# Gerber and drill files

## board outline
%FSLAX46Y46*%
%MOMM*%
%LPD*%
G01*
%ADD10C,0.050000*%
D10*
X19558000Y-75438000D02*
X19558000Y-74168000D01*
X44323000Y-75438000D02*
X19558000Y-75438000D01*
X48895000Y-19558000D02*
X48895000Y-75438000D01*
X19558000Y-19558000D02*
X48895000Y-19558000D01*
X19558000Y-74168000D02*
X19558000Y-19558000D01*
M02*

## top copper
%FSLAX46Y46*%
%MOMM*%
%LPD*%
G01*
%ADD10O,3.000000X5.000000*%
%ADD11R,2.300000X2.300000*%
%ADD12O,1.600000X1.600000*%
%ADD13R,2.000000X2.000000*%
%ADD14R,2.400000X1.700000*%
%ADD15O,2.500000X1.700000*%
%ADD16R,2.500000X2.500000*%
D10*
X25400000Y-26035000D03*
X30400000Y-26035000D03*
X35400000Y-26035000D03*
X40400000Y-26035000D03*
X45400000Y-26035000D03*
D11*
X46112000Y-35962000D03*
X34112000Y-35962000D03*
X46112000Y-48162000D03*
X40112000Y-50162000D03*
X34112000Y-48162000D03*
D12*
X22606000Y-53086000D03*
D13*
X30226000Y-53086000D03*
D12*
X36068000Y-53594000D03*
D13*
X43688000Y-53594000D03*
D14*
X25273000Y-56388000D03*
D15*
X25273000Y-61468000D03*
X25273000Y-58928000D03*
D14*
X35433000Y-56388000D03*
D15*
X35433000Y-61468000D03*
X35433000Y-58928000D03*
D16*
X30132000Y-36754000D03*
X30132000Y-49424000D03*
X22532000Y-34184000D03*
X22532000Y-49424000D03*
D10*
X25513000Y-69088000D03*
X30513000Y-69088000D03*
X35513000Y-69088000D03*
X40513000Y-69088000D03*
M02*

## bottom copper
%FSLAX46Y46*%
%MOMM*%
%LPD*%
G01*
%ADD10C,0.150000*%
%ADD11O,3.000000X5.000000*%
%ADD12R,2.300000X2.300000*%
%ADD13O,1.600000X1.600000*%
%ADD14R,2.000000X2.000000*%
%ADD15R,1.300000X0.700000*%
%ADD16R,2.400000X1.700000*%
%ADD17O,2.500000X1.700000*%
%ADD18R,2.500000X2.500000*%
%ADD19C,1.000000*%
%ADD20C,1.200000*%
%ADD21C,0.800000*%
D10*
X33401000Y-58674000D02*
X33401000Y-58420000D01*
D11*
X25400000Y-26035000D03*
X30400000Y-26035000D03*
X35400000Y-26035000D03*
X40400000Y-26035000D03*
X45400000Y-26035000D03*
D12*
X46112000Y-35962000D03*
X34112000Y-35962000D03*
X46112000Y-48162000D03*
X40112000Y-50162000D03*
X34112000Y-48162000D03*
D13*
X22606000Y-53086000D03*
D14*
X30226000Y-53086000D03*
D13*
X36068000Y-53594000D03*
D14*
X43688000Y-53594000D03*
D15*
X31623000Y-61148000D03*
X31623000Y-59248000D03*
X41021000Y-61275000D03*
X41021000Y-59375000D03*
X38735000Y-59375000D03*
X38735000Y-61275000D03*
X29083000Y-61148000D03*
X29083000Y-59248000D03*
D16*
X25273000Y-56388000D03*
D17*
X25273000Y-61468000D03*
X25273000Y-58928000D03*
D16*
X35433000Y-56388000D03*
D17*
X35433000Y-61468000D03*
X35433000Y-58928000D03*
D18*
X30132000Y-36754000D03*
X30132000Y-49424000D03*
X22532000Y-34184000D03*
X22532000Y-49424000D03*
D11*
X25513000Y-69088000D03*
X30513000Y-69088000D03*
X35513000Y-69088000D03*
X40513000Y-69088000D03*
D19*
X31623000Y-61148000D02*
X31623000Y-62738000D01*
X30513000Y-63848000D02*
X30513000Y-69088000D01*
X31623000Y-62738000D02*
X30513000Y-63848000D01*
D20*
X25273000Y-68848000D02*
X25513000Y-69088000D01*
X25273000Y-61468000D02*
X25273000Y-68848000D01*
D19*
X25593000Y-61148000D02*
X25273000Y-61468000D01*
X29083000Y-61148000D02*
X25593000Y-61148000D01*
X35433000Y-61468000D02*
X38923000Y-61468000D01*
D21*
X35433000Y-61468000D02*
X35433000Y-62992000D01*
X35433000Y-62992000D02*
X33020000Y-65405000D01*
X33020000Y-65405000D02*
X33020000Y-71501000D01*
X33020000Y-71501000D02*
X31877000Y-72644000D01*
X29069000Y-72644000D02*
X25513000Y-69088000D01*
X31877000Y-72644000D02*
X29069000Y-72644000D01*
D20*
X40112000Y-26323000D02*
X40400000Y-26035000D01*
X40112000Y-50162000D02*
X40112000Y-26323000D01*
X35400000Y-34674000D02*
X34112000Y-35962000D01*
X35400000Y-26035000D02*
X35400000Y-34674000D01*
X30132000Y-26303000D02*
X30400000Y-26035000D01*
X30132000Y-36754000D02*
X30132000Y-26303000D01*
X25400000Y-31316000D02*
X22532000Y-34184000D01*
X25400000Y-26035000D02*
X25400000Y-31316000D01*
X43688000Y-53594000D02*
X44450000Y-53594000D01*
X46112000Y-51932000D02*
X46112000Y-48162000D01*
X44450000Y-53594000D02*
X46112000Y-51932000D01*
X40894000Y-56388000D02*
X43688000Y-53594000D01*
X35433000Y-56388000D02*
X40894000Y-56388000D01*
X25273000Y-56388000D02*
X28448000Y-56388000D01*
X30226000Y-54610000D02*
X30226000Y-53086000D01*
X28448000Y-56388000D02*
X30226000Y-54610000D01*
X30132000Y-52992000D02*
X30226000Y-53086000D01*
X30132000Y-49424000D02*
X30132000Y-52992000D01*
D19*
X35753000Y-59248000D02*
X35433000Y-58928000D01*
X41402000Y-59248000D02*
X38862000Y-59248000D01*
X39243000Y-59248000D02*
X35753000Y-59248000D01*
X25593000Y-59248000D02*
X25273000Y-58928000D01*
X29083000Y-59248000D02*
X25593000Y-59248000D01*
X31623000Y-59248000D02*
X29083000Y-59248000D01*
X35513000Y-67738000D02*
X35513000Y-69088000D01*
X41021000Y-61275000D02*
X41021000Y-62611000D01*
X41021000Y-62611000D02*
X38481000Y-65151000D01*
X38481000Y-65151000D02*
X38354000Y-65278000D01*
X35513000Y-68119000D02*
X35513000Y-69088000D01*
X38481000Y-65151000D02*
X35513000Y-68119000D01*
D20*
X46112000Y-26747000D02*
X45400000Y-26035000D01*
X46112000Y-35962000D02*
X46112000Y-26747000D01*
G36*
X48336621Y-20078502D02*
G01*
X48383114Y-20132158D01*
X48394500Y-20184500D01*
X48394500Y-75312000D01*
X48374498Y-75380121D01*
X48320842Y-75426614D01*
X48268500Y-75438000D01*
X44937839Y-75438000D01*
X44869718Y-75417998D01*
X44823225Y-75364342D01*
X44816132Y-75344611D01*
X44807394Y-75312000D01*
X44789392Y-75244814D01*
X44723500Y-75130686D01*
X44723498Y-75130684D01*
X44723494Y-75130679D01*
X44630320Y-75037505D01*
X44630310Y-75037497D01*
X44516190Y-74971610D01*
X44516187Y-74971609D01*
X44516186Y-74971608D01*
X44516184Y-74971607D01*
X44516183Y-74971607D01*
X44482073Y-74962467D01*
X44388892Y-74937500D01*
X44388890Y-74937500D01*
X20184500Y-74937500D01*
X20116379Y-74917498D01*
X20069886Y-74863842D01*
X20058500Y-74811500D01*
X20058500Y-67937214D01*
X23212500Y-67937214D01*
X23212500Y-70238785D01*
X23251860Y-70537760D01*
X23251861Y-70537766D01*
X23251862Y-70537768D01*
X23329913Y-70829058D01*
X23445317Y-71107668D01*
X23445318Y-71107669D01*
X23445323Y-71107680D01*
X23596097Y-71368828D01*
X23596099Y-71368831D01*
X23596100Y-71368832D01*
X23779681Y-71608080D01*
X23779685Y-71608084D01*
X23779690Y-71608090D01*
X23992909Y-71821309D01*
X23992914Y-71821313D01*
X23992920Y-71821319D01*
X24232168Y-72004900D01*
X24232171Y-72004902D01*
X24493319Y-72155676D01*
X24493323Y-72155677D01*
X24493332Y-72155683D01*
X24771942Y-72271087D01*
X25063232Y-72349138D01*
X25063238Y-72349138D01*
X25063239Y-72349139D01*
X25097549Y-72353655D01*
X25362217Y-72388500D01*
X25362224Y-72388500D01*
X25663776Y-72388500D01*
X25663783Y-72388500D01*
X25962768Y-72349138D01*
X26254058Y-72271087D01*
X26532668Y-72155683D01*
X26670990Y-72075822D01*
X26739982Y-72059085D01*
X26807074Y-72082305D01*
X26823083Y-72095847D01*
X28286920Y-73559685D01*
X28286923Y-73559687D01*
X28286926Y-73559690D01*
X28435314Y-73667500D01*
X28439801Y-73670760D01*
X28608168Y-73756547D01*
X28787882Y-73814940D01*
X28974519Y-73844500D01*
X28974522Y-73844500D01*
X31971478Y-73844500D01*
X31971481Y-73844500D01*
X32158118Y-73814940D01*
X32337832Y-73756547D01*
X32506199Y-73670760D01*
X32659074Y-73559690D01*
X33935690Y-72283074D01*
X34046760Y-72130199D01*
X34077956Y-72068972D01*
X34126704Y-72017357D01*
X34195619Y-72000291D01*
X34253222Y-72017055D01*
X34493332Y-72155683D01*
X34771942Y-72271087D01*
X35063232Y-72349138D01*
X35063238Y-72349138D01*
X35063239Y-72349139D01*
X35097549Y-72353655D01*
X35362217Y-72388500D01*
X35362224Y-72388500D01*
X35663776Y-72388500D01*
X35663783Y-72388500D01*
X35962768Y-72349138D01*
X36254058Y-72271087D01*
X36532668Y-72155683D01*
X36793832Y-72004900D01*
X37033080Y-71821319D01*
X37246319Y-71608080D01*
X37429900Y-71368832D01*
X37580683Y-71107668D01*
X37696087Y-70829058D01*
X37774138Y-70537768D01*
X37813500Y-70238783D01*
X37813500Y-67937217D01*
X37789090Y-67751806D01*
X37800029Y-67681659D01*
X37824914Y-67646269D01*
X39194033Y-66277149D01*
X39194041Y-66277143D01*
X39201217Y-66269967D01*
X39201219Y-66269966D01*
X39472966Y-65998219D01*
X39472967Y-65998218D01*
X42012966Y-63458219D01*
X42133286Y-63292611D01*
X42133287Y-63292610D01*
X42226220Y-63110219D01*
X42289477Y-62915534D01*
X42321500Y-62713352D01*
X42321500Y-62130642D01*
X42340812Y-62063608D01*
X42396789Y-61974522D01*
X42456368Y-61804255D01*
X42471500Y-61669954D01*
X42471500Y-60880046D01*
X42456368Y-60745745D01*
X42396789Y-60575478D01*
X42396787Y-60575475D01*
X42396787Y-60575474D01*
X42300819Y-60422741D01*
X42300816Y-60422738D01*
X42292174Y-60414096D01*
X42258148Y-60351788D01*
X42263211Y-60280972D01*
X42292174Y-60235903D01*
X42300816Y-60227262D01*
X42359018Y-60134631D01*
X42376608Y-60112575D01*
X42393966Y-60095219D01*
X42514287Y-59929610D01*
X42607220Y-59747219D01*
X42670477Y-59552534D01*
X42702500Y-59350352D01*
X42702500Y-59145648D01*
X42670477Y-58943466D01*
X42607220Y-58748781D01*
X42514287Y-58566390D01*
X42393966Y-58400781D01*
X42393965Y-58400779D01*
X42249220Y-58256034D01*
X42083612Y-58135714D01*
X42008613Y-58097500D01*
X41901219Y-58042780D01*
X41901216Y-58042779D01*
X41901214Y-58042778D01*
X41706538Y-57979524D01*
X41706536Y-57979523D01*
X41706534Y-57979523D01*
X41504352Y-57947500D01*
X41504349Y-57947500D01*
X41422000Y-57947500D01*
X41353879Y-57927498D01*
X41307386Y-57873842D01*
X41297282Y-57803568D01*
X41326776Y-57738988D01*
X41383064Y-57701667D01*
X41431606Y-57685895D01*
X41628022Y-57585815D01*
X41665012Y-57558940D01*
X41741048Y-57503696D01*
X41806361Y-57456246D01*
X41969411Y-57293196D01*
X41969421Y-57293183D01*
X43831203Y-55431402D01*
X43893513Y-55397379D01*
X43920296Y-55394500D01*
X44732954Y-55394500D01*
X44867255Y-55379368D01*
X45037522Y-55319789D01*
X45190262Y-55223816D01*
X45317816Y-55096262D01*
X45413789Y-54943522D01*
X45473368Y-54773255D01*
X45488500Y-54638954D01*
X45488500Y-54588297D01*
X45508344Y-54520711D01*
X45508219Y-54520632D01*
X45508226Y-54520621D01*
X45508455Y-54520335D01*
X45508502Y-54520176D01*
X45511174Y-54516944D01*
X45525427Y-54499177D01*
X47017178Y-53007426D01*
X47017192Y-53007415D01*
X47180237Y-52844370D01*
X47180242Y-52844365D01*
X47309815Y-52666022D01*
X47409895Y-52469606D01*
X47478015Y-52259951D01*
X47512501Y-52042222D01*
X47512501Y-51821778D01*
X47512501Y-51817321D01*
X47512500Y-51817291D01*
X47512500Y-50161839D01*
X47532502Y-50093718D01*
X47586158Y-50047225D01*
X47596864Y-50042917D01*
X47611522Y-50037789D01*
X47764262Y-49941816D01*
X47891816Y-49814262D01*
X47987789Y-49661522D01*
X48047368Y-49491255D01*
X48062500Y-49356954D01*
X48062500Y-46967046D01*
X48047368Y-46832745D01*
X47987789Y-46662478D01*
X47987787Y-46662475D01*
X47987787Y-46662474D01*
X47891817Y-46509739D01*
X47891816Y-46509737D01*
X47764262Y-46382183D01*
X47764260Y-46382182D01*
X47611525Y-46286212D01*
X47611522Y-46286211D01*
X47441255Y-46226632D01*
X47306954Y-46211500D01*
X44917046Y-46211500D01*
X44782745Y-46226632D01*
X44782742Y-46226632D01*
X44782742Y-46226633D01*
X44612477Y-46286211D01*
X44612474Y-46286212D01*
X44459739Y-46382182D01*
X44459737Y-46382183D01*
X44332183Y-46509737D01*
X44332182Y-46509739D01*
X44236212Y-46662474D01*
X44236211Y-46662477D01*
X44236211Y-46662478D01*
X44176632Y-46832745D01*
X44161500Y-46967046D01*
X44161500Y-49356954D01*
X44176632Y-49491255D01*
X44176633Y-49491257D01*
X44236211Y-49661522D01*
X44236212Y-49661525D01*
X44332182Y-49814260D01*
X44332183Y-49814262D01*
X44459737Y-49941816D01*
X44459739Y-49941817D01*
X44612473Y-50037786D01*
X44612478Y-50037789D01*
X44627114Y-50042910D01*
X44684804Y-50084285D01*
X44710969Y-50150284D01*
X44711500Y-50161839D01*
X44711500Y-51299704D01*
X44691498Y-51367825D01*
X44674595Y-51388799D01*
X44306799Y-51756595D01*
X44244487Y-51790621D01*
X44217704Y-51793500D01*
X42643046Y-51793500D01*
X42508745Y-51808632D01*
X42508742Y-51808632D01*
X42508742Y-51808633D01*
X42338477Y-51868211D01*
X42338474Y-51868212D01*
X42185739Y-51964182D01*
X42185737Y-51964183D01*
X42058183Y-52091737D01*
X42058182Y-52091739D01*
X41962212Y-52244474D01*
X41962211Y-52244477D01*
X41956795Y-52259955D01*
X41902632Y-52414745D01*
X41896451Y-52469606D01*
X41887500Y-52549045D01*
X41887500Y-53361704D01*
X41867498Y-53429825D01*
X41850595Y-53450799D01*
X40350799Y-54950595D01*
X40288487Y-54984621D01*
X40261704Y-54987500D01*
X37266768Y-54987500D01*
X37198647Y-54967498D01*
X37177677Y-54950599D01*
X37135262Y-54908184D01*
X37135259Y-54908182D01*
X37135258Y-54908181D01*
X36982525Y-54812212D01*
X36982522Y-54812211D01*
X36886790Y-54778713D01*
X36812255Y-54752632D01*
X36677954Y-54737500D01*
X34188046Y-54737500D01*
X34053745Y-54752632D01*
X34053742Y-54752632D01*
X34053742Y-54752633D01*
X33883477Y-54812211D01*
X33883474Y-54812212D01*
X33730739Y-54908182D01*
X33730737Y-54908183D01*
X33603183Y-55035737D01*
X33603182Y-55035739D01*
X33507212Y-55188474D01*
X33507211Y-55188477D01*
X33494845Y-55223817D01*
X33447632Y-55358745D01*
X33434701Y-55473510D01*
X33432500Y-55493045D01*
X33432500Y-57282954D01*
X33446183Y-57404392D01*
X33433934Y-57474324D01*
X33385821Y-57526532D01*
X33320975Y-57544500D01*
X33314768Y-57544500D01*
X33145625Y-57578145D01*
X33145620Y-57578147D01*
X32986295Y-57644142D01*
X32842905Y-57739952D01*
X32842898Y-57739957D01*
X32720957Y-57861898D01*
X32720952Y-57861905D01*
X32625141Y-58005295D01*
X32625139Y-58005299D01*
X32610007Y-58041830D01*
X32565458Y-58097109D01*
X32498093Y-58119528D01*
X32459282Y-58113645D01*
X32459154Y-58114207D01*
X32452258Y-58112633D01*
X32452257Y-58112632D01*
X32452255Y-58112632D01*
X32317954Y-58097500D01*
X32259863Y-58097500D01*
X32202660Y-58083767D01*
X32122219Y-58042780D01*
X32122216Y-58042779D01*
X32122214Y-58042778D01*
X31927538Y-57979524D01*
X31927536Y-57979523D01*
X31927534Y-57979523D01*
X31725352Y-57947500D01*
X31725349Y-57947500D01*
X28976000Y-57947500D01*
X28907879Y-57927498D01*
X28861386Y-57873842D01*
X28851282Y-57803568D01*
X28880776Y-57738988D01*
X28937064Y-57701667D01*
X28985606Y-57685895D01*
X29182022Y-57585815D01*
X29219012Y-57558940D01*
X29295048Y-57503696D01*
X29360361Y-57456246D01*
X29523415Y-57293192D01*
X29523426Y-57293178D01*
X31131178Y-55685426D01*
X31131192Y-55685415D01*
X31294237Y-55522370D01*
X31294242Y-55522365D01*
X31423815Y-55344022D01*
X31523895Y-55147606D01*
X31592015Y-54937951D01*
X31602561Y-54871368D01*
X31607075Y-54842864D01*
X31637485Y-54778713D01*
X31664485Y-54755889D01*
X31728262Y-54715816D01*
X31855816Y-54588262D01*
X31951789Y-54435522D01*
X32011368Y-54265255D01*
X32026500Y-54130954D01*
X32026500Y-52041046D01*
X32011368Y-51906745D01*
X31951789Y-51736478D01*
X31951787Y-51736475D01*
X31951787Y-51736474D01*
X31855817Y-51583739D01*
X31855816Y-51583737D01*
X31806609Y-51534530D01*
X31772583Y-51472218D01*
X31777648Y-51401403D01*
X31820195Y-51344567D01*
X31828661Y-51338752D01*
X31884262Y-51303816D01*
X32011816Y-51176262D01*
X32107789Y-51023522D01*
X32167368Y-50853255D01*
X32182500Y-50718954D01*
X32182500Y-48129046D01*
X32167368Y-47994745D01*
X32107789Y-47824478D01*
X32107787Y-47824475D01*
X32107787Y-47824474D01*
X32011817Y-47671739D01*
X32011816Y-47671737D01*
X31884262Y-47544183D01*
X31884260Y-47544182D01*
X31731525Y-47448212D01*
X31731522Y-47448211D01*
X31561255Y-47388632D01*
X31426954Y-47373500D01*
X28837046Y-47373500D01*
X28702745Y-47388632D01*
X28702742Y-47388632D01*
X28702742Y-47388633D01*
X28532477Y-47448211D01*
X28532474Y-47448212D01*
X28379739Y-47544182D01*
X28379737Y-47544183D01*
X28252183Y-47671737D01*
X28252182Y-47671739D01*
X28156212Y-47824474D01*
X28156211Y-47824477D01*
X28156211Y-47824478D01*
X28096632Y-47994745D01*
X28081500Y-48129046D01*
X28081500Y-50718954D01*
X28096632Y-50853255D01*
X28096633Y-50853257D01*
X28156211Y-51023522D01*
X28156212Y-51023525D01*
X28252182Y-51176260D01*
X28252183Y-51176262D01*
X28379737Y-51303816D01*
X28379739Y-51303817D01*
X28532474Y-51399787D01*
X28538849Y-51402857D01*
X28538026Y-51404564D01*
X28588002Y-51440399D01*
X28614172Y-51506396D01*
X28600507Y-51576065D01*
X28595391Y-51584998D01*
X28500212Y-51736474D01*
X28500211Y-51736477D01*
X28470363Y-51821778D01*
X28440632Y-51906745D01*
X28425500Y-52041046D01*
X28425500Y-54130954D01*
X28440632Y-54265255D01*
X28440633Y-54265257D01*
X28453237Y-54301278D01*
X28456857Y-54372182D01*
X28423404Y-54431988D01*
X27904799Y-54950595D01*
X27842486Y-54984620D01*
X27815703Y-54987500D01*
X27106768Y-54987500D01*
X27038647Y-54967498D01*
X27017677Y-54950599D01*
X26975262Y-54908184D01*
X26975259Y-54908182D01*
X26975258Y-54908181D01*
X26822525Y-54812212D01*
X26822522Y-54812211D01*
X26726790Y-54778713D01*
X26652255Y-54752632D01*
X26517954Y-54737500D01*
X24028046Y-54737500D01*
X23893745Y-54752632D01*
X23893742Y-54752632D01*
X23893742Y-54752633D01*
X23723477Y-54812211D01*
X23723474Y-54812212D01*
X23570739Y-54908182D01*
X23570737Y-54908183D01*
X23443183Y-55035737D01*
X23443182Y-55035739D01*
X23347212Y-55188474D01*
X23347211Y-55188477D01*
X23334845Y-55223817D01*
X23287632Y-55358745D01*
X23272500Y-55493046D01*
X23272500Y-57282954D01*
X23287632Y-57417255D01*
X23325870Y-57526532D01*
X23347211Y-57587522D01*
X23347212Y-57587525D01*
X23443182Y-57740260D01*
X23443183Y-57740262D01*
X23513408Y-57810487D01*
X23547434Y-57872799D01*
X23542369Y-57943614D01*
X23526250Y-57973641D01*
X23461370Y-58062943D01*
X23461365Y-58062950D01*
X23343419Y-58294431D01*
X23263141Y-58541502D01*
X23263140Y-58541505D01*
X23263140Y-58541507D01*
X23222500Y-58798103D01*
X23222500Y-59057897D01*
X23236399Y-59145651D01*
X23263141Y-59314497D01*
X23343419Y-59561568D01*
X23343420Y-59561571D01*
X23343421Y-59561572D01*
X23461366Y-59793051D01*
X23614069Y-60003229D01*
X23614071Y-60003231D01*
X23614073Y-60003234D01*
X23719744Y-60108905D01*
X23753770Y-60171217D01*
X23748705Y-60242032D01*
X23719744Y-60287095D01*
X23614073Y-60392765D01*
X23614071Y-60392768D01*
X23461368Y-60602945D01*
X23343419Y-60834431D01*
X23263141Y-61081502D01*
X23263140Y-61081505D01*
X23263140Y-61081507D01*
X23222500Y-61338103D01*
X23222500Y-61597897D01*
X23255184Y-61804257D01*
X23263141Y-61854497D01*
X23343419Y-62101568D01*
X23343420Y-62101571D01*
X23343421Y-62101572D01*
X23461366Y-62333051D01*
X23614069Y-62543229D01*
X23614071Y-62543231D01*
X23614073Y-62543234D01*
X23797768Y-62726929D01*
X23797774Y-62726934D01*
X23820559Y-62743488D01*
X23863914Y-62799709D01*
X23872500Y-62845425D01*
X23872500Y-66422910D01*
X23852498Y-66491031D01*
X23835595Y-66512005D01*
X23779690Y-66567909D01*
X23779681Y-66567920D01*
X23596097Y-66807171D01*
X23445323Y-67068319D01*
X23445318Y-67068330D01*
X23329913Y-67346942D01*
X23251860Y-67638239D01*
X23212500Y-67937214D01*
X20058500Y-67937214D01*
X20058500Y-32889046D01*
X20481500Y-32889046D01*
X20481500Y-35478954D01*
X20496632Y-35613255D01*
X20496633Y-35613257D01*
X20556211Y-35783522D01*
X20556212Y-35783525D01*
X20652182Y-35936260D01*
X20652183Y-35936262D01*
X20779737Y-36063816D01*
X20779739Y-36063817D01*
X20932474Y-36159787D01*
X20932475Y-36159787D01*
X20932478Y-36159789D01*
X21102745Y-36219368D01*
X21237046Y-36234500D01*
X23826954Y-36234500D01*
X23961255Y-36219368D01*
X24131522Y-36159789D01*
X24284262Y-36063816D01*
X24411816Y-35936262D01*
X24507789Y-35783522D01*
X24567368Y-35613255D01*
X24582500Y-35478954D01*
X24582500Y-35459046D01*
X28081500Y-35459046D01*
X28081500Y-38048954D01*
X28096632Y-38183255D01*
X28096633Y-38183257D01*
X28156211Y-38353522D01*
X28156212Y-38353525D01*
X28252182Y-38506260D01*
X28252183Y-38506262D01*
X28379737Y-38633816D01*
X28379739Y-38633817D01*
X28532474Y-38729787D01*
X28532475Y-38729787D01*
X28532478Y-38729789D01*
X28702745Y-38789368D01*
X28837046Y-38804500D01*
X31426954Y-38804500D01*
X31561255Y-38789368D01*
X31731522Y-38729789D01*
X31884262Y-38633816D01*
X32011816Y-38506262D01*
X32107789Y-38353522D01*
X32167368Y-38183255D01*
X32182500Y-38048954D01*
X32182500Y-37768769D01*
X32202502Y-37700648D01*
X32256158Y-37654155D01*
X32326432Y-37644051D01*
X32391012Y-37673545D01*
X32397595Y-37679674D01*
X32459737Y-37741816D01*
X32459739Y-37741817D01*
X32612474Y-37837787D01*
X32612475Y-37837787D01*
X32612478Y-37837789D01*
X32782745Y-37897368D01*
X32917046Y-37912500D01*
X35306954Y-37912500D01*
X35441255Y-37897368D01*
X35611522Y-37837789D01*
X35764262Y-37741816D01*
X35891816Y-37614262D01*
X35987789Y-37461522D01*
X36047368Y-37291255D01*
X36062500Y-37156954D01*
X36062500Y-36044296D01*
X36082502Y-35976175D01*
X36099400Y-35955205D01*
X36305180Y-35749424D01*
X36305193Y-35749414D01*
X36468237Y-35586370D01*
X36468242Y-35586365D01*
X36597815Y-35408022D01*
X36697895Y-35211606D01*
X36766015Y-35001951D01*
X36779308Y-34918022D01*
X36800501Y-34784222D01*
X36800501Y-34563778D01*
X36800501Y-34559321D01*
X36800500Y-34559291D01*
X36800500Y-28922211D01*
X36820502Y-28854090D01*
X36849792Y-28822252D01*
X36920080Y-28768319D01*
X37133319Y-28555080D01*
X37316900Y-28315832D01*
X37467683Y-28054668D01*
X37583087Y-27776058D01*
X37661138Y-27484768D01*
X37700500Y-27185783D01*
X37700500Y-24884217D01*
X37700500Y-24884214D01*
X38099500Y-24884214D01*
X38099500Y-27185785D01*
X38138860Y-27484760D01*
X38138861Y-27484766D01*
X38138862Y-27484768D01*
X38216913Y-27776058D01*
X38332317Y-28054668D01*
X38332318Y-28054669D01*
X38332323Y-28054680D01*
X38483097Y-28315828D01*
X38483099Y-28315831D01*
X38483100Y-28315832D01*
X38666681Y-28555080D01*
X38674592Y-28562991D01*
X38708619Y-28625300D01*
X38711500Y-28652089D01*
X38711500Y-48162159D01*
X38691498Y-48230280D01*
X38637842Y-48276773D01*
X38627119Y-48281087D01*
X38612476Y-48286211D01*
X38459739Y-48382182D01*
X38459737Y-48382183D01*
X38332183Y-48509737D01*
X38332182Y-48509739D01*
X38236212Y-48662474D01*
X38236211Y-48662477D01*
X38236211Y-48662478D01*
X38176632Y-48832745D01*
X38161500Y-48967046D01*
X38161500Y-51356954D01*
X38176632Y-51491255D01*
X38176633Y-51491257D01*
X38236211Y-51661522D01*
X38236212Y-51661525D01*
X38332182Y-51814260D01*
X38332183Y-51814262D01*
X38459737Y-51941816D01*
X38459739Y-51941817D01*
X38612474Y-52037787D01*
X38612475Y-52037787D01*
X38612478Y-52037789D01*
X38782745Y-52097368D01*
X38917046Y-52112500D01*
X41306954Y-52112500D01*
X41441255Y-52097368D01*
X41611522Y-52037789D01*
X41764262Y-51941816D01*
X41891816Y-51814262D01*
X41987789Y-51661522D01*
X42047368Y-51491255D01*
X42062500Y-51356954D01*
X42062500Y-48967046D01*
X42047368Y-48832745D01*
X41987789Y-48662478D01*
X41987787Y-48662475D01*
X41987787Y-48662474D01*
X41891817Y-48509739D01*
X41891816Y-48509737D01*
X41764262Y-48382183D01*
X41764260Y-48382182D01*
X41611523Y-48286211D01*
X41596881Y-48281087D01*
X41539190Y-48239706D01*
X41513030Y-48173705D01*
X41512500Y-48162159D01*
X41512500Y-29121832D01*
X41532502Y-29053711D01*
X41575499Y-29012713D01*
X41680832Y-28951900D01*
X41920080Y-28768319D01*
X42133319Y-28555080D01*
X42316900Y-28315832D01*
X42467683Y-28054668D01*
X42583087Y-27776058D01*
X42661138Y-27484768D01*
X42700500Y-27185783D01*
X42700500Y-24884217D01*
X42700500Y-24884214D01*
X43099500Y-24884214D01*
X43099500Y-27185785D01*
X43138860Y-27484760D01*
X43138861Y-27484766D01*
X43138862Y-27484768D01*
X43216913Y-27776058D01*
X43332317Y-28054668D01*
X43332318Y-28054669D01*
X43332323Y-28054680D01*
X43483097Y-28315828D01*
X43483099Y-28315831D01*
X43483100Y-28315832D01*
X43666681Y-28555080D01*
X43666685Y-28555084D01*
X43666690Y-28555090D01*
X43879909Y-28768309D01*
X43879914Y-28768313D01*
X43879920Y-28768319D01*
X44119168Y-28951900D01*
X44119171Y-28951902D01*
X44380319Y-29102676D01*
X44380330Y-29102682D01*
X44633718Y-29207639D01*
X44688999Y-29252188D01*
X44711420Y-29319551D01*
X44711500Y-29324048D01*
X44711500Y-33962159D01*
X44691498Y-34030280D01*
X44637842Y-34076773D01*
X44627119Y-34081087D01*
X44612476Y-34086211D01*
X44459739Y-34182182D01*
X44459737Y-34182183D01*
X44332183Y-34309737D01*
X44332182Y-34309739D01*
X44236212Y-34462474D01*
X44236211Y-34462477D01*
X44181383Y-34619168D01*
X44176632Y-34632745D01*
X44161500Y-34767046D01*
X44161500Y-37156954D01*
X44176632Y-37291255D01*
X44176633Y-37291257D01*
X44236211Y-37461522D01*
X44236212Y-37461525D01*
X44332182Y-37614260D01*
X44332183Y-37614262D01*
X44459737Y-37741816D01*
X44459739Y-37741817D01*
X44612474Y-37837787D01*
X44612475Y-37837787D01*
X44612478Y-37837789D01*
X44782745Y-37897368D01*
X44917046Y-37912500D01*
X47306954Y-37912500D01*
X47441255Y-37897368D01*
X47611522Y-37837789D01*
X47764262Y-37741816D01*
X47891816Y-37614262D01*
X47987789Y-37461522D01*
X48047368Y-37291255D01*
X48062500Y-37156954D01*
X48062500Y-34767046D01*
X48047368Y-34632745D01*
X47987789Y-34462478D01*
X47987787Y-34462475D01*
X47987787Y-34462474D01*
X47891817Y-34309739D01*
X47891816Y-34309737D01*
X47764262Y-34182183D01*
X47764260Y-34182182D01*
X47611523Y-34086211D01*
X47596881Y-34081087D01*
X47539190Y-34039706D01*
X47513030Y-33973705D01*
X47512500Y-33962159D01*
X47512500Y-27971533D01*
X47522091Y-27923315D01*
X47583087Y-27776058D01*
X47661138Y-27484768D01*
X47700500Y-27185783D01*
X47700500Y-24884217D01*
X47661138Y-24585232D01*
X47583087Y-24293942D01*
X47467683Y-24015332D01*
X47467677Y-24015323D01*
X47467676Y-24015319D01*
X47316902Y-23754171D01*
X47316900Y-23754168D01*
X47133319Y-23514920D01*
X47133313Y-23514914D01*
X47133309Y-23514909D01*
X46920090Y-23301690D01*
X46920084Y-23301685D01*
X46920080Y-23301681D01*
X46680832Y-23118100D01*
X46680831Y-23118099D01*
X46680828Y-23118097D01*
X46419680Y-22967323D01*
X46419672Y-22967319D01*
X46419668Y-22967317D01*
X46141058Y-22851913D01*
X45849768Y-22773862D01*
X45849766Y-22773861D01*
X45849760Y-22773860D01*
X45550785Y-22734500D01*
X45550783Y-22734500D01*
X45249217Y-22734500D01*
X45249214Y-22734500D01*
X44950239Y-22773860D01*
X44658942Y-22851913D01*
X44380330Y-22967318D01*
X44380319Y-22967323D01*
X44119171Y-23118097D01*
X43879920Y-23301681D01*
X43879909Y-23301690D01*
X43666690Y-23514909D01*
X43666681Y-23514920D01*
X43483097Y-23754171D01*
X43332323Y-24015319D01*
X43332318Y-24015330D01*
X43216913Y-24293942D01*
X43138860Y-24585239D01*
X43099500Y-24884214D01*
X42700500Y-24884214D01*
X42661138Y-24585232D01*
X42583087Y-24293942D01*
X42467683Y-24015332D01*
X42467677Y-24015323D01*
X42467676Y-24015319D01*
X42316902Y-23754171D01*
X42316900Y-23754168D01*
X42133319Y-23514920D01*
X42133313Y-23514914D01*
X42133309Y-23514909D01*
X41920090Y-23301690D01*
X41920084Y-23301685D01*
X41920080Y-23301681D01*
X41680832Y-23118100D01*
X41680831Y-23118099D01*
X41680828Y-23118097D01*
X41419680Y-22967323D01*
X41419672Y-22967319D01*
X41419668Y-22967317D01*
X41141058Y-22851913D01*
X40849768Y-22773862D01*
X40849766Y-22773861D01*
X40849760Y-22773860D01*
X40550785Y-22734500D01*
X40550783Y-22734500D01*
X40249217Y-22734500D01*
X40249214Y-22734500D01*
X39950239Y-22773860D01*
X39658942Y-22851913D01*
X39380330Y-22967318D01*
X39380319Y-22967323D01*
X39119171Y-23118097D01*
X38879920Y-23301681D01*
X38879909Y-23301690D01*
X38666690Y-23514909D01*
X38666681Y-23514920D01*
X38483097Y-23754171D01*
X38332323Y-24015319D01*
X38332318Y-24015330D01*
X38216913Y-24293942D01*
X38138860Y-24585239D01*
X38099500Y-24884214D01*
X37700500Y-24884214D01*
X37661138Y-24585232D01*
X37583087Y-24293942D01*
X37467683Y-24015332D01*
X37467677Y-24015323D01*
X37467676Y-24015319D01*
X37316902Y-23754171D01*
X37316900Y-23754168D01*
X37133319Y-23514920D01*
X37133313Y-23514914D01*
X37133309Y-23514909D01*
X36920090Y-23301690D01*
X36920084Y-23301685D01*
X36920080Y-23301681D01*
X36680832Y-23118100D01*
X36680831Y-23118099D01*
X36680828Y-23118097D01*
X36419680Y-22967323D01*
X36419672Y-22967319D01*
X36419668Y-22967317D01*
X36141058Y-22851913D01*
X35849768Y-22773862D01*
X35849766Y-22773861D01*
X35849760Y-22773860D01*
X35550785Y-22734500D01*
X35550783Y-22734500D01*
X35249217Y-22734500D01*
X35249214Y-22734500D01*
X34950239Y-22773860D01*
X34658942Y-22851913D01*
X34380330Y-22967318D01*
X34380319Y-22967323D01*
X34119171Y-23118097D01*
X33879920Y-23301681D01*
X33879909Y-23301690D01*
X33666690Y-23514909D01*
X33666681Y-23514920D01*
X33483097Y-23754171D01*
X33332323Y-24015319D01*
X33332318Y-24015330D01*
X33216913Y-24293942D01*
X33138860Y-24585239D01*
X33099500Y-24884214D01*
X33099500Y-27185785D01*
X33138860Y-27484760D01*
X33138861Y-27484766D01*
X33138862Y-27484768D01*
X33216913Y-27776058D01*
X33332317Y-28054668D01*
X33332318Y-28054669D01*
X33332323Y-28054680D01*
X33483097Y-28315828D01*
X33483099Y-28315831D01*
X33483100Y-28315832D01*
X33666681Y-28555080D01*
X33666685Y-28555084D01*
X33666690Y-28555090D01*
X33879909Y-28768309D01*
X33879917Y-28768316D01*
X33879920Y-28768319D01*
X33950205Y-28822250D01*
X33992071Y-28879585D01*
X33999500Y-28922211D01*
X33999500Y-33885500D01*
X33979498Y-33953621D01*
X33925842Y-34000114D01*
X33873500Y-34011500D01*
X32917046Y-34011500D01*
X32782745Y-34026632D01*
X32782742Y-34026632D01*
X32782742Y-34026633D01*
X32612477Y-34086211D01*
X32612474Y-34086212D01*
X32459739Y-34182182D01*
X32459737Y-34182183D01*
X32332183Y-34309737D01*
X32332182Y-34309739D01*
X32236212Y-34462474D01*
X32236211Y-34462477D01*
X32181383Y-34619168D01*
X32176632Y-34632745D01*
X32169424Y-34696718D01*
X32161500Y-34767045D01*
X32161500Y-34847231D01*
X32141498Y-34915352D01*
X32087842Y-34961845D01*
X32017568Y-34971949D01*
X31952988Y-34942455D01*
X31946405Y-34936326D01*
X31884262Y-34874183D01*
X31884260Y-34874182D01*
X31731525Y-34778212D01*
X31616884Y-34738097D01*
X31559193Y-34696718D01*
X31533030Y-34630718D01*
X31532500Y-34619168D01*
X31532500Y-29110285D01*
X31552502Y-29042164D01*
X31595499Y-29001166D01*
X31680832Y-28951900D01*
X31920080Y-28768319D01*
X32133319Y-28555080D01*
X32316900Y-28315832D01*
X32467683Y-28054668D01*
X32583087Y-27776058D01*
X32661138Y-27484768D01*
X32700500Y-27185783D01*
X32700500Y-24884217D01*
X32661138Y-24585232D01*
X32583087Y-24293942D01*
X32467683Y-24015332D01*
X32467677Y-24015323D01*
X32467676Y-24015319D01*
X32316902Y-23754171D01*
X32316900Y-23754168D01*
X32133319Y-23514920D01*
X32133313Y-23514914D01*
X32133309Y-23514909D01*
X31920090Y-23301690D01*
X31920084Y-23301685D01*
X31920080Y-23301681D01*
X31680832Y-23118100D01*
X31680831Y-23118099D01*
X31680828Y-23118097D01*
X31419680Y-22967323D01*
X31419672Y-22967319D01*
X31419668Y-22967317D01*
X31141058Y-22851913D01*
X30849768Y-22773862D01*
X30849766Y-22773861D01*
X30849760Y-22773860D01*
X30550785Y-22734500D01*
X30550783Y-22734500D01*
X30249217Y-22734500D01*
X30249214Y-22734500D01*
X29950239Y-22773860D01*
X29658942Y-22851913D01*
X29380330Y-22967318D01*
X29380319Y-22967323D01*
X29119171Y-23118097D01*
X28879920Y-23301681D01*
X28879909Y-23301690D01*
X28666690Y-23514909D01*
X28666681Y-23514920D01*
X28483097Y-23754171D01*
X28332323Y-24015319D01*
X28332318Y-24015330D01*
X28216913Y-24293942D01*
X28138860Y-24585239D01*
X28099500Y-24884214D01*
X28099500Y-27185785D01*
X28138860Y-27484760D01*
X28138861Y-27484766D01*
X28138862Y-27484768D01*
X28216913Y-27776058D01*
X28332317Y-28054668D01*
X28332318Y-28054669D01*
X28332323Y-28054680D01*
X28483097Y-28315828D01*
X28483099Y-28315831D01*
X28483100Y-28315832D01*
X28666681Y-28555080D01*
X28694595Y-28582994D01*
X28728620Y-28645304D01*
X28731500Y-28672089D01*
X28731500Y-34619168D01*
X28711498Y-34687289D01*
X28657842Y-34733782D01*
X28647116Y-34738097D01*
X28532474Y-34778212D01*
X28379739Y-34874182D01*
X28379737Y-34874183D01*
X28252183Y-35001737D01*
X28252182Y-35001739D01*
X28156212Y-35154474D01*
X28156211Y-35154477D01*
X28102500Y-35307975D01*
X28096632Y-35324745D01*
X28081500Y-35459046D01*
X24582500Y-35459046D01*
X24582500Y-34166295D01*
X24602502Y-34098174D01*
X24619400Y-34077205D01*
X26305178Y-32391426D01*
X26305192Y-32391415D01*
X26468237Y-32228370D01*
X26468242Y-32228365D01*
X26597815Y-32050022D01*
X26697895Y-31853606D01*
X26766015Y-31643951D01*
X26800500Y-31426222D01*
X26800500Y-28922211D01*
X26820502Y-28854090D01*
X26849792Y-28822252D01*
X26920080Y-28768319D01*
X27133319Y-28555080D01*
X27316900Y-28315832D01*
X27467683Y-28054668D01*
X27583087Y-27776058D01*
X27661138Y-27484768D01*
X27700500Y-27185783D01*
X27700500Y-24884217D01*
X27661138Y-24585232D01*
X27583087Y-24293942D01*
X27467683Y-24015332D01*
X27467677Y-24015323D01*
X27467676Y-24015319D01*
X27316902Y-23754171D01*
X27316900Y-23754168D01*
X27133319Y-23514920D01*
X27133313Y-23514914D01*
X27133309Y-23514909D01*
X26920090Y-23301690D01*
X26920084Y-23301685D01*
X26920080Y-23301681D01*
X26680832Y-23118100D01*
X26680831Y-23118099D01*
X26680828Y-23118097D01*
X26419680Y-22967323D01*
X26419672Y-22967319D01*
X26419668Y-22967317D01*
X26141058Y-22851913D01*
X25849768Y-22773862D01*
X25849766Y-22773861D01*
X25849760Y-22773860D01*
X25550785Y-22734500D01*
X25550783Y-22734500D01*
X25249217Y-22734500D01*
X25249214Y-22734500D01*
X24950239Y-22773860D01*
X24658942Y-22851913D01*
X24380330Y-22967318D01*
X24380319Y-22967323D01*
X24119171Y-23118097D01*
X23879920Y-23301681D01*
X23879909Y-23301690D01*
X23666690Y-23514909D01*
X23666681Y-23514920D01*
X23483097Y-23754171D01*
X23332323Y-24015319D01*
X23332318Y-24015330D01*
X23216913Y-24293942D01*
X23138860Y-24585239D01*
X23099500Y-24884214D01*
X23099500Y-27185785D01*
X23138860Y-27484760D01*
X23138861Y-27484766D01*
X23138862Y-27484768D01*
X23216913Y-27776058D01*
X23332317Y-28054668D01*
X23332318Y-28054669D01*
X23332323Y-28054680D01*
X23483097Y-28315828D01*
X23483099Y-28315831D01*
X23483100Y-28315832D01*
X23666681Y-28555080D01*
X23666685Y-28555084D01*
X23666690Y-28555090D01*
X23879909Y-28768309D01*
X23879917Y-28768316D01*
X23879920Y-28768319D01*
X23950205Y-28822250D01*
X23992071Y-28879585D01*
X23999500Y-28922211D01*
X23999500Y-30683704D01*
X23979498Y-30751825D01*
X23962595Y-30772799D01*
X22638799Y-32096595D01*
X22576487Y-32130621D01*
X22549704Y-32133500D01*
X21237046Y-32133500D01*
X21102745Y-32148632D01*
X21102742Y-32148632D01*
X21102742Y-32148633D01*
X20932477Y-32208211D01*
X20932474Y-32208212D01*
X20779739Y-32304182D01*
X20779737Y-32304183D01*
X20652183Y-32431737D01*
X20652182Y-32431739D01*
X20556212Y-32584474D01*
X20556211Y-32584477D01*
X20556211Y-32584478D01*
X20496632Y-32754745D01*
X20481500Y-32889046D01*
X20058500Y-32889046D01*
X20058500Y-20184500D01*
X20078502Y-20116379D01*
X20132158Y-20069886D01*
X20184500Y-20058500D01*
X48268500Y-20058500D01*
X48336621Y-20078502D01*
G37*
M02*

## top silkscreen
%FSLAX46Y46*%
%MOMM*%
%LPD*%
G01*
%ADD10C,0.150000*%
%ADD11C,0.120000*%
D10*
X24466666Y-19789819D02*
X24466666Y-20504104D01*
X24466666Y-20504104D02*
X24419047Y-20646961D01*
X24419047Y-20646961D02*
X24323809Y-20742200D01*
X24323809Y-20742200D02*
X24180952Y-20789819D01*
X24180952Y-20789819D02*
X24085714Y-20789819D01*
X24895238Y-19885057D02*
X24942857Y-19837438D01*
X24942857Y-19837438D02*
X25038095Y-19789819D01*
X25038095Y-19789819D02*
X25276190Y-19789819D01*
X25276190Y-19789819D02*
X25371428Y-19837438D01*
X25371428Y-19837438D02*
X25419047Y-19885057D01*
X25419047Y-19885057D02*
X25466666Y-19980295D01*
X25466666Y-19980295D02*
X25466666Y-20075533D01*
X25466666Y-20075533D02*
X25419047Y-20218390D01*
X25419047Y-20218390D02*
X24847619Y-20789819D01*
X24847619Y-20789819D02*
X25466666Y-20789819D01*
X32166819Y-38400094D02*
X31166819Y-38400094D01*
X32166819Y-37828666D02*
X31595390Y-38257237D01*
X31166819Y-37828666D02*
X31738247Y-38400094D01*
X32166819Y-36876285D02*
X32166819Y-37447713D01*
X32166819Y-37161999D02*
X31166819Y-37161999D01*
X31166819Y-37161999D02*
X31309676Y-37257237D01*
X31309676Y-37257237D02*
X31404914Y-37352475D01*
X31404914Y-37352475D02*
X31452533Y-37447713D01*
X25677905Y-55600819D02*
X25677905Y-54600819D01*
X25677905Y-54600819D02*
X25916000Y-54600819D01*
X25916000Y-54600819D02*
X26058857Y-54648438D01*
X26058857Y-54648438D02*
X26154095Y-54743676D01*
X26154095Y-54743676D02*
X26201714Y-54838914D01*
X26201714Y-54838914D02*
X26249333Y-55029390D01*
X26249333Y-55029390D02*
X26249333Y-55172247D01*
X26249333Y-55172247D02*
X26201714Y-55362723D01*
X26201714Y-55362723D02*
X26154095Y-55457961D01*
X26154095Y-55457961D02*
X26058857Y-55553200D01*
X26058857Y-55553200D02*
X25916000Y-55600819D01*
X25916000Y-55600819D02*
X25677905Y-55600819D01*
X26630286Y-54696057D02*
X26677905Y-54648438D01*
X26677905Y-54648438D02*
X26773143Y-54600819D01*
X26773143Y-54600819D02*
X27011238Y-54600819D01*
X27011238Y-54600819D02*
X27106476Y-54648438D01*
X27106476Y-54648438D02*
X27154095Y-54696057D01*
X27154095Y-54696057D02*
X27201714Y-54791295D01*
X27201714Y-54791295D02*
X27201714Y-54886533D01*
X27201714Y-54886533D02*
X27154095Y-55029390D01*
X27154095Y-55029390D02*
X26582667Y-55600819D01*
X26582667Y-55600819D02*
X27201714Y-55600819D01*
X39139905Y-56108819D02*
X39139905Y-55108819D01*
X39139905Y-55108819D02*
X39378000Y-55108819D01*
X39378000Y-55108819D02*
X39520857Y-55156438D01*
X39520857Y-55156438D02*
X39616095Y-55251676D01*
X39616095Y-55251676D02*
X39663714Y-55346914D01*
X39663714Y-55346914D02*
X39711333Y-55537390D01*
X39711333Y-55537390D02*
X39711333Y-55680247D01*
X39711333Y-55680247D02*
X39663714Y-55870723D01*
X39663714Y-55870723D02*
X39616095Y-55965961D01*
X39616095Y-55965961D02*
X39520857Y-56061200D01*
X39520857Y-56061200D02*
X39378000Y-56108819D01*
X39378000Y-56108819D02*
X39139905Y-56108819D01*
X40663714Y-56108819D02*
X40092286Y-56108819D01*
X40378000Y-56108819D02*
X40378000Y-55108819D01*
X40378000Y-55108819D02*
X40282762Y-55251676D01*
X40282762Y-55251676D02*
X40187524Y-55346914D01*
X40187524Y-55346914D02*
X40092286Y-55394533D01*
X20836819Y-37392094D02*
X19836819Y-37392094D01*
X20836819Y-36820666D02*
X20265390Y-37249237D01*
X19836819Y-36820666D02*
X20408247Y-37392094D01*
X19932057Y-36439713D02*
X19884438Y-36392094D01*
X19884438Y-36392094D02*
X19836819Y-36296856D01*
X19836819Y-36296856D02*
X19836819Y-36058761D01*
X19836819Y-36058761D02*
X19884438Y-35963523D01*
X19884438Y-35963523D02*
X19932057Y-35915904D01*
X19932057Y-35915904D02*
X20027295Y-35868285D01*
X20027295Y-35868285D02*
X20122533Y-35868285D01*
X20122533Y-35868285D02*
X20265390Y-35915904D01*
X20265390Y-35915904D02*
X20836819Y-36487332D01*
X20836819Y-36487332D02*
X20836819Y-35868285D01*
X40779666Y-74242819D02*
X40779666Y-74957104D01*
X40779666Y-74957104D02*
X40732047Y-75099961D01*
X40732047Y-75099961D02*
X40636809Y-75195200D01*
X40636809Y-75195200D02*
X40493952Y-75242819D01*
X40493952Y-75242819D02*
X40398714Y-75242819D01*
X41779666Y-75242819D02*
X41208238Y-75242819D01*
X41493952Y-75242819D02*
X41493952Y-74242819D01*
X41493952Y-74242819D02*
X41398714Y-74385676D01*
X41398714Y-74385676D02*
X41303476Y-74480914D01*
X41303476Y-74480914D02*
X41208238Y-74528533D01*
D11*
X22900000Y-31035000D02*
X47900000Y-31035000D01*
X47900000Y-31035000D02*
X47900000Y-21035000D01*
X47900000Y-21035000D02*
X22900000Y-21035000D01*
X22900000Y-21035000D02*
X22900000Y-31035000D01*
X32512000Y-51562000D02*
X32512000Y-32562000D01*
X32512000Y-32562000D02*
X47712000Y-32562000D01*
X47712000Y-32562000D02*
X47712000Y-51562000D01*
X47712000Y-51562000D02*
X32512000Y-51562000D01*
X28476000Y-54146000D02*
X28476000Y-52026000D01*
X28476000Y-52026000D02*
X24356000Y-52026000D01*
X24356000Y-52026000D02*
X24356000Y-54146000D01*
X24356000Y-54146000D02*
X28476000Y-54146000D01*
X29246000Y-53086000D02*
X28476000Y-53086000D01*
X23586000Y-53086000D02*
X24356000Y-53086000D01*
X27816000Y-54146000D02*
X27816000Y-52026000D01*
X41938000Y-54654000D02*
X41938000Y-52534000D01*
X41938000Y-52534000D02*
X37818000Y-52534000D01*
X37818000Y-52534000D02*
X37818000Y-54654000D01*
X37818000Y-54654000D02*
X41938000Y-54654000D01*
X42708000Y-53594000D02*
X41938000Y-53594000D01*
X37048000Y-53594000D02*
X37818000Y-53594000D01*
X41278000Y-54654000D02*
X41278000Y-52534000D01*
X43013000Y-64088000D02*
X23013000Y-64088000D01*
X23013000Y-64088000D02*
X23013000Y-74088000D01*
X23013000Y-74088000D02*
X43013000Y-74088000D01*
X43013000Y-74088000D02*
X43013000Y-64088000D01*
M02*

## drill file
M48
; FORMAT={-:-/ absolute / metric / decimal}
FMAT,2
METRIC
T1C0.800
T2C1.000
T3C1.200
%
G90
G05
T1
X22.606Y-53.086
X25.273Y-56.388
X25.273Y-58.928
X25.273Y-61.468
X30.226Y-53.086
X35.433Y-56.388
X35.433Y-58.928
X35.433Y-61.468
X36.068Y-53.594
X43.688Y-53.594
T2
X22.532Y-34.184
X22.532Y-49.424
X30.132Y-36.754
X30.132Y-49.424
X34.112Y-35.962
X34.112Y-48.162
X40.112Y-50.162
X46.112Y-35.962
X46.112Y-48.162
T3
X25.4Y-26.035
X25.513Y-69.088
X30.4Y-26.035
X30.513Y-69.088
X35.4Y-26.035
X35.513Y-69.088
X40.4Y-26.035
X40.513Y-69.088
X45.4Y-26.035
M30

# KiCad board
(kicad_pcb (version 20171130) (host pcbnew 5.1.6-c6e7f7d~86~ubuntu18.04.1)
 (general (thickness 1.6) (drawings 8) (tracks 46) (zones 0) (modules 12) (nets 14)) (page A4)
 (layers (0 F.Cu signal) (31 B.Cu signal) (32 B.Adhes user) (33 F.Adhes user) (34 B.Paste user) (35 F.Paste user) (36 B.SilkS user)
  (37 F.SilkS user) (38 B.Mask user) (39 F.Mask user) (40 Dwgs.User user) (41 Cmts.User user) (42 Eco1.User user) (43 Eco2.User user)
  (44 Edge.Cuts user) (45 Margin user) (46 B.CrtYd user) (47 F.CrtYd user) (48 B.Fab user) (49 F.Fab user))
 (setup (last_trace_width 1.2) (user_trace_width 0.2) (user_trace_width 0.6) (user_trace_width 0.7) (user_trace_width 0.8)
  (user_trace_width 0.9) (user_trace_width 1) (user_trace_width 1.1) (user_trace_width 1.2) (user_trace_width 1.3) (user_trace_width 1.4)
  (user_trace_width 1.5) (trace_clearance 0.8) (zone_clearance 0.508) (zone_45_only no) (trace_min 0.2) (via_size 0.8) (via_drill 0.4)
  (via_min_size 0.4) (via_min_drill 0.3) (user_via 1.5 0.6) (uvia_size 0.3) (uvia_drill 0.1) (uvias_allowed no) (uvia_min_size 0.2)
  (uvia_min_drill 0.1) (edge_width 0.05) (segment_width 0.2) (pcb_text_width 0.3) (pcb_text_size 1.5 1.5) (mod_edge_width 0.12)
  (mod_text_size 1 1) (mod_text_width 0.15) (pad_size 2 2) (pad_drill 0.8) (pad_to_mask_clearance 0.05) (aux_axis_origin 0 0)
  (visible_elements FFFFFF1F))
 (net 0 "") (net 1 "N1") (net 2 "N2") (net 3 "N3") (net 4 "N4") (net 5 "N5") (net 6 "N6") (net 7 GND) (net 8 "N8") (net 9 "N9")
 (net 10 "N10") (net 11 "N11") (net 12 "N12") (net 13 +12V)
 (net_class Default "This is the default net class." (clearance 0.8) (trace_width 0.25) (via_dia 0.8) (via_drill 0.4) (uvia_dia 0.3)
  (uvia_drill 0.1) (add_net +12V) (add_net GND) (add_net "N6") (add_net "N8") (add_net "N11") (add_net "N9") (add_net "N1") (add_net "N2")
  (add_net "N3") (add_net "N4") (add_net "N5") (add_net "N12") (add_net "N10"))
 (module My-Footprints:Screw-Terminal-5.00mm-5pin (layer F.Cu) (at 25.4 26.035)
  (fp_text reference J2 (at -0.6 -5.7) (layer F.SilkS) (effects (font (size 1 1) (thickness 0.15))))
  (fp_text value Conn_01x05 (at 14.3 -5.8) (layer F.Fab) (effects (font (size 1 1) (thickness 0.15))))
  (fp_line (start -2.5 5) (end 22.5 5) (layer F.SilkS) (width 0.12))
  (fp_line (start 22.5 5) (end 22.5 -5) (layer F.SilkS) (width 0.12))
  (fp_line (start 22.5 -5) (end -2.5 -5) (layer F.SilkS) (width 0.12))
  (fp_line (start -2.5 -5) (end -2.5 5) (layer F.SilkS) (width 0.12))
  (pad 1 thru_hole oval (at 0 0 90) (size 5 3) (drill 1.2) (layers *.Cu *.Mask) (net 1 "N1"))
  (pad 2 thru_hole oval (at 5 0 90) (size 5 3) (drill 1.2) (layers *.Cu *.Mask) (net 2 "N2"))
  (pad 3 thru_hole oval (at 10 0 90) (size 5 3) (drill 1.2) (layers *.Cu *.Mask) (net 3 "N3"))
  (pad 4 thru_hole oval (at 15 0 90) (size 5 3) (drill 1.2) (layers *.Cu *.Mask) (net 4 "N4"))
  (pad 5 thru_hole oval (at 20 0 90) (size 5 3) (drill 1.2) (layers *.Cu *.Mask) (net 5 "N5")))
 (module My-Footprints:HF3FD (layer F.Cu) (at 32.512 51.562 90)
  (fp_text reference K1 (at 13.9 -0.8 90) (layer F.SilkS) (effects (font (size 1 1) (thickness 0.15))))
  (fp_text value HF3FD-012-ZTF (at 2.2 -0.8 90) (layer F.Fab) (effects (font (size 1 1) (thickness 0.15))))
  (fp_line (start 0 0) (end 19 0) (layer F.SilkS) (width 0.12))
  (fp_line (start 19 0) (end 19 15.2) (layer F.SilkS) (width 0.12))
  (fp_line (start 19 15.2) (end 0 15.2) (layer F.SilkS) (width 0.12))
  (fp_line (start 0 15.2) (end 0 0) (layer F.SilkS) (width 0.12))
  (pad NC thru_hole rect (at 15.6 13.6 90) (size 2.3 2.3) (drill 1) (layers *.Cu *.Mask) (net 5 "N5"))
  (pad NO thru_hole rect (at 15.6 1.6 90) (size 2.3 2.3) (drill 1) (layers *.Cu *.Mask) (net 3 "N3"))
  (pad C2 thru_hole rect (at 3.4 13.6 90) (size 2.3 2.3) (drill 1) (layers *.Cu *.Mask) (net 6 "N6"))
  (pad COM thru_hole rect (at 1.4 7.6 90) (size 2.3 2.3) (drill 1) (layers *.Cu *.Mask) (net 4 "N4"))
  (pad C1 thru_hole rect (at 3.4 1.6 90) (size 2.3 2.3) (drill 1) (layers *.Cu *.Mask) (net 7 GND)))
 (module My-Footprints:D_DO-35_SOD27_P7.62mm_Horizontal (layer F.Cu) (at 30.226 53.086 180)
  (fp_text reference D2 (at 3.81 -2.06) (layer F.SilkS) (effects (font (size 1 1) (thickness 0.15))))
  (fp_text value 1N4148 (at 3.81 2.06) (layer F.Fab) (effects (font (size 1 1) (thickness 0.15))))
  (fp_line (start 1.75 -1.06) (end 1.75 1.06) (layer F.SilkS) (width 0.12))
  (fp_line (start 1.75 1.06) (end 5.87 1.06) (layer F.SilkS) (width 0.12))
  (fp_line (start 5.87 1.06) (end 5.87 -1.06) (layer F.SilkS) (width 0.12))
  (fp_line (start 5.87 -1.06) (end 1.75 -1.06) (layer F.SilkS) (width 0.12))
  (fp_line (start 0.98 0) (end 1.75 0) (layer F.SilkS) (width 0.12))
  (fp_line (start 6.64 0) (end 5.87 0) (layer F.SilkS) (width 0.12))
  (fp_line (start 2.41 -1.06) (end 2.41 1.06) (layer F.SilkS) (width 0.12))
  (pad A thru_hole oval (at 7.62 0 180) (size 1.6 1.6) (drill 0.8) (layers *.Cu *.Mask) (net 7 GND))
  (pad C thru_hole rect (at 0 0 180) (size 2 2) (drill 0.8) (layers *.Cu *.Mask) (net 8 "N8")))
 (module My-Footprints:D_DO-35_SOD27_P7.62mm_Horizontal (layer F.Cu) (at 43.688 53.594 180)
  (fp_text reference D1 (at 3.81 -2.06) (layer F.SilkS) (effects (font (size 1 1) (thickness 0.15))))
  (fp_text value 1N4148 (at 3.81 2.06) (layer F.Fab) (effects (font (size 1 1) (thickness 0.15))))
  (fp_line (start 1.75 -1.06) (end 1.75 1.06) (layer F.SilkS) (width 0.12))
  (fp_line (start 1.75 1.06) (end 5.87 1.06) (layer F.SilkS) (width 0.12))
  (fp_line (start 5.87 1.06) (end 5.87 -1.06) (layer F.SilkS) (width 0.12))
  (fp_line (start 5.87 -1.06) (end 1.75 -1.06) (layer F.SilkS) (width 0.12))
  (fp_line (start 0.98 0) (end 1.75 0) (layer F.SilkS) (width 0.12))
  (fp_line (start 6.64 0) (end 5.87 0) (layer F.SilkS) (width 0.12))
  (fp_line (start 2.41 -1.06) (end 2.41 1.06) (layer F.SilkS) (width 0.12))
  (pad A thru_hole oval (at 7.62 0 180) (size 1.6 1.6) (drill 0.8) (layers *.Cu *.Mask) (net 7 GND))
  (pad C thru_hole rect (at 0 0 180) (size 2 2) (drill 0.8) (layers *.Cu *.Mask) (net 6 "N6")))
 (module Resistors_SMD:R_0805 (layer B.Cu) (at 31.623 60.198 90)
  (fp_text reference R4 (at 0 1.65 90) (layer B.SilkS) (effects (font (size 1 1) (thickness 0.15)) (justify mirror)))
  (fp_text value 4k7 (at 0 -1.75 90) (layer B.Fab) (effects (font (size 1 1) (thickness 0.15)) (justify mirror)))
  (pad 1 smd rect (at -0.95 0 90) (size 0.7 1.3) (layers B.Cu B.Paste B.Mask) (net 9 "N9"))
  (pad 2 smd rect (at 0.95 0 90) (size 0.7 1.3) (layers B.Cu B.Paste B.Mask) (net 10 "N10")))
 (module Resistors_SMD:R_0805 (layer B.Cu) (at 41.021 60.325 90)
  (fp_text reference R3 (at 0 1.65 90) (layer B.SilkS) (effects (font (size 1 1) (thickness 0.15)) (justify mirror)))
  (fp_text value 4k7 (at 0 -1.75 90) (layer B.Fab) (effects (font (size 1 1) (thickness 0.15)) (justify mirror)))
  (pad 1 smd rect (at -0.95 0 90) (size 0.7 1.3) (layers B.Cu B.Paste B.Mask) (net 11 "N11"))
  (pad 2 smd rect (at 0.95 0 90) (size 0.7 1.3) (layers B.Cu B.Paste B.Mask) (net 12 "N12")))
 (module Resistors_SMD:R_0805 (layer B.Cu) (at 38.735 60.325 270)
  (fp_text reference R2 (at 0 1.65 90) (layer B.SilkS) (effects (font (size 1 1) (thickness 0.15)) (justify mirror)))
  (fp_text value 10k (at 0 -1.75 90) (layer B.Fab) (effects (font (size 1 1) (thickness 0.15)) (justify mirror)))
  (pad 1 smd rect (at -0.95 0 270) (size 0.7 1.3) (layers B.Cu B.Paste B.Mask) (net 12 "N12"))
  (pad 2 smd rect (at 0.95 0 270) (size 0.7 1.3) (layers B.Cu B.Paste B.Mask) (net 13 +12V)))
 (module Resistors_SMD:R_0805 (layer B.Cu) (at 29.083 60.198 90)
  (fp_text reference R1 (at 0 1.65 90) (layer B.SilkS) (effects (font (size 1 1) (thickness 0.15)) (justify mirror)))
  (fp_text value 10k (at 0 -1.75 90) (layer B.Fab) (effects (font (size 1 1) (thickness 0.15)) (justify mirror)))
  (pad 1 smd rect (at -0.95 0 90) (size 0.7 1.3) (layers B.Cu B.Paste B.Mask) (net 13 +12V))
  (pad 2 smd rect (at 0.95 0 90) (size 0.7 1.3) (layers B.Cu B.Paste B.Mask) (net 10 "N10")))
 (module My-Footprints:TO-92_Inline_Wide (layer B.Cu) (at 25.273 56.388 270)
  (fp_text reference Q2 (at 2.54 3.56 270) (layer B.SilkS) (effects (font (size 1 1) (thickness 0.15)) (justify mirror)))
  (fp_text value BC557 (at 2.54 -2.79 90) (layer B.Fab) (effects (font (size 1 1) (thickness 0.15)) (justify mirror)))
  (pad 1 thru_hole rect (at 0 0 180) (size 2.4 1.7) (drill 0.8) (layers *.Cu *.Mask) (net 8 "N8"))
  (pad 3 thru_hole oval (at 5.08 0 180) (size 2.5 1.7) (drill 0.8) (layers *.Cu *.Mask) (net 13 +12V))
  (pad 2 thru_hole oval (at 2.54 0 180) (size 2.5 1.7) (drill 0.8) (layers *.Cu *.Mask) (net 10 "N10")))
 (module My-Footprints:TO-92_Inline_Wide (layer B.Cu) (at 35.433 56.388 270)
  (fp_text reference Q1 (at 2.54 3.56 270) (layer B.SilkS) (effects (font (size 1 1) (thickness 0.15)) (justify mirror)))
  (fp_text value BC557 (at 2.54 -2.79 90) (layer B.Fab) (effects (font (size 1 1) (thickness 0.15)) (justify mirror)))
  (pad 1 thru_hole rect (at 0 0 180) (size 2.4 1.7) (drill 0.8) (layers *.Cu *.Mask) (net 6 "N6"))
  (pad 3 thru_hole oval (at 5.08 0 180) (size 2.5 1.7) (drill 0.8) (layers *.Cu *.Mask) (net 13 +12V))
  (pad 2 thru_hole oval (at 2.54 0 180) (size 2.5 1.7) (drill 0.8) (layers *.Cu *.Mask) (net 12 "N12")))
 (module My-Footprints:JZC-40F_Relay (layer F.Cu) (at 21.082 51.054 90)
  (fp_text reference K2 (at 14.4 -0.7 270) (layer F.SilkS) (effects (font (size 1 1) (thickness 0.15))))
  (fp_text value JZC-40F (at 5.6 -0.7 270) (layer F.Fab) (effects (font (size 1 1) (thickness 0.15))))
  (pad 4 thru_hole rect (at 14.3 9.05 90) (size 2.5 2.5) (drill 1) (layers *.Cu *.Mask) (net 2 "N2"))
  (pad 1 thru_hole rect (at 1.63 9.05 90) (size 2.5 2.5) (drill 1) (layers *.Cu *.Mask) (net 8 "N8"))
  (pad 3 thru_hole rect (at 16.87 1.45 90) (size 2.5 2.5) (drill 1) (layers *.Cu *.Mask) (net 1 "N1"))
  (pad 2 thru_hole rect (at 1.63 1.45 90) (size 2.5 2.5) (drill 1) (layers *.Cu *.Mask) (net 7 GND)))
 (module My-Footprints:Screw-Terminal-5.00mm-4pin (layer F.Cu) (at 40.513 69.088 180)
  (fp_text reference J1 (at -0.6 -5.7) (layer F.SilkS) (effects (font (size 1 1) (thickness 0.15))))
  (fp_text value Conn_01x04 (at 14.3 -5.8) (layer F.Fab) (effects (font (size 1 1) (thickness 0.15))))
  (fp_line (start -2.5 5) (end 17.5 5) (layer F.SilkS) (width 0.12))
  (fp_line (start 17.5 5) (end 17.5 -5) (layer F.SilkS) (width 0.12))
  (fp_line (start 17.5 -5) (end -2.5 -5) (layer F.SilkS) (width 0.12))
  (fp_line (start -2.5 -5) (end -2.5 5) (layer F.SilkS) (width 0.12))
  (pad 4 thru_hole oval (at 15 0 270) (size 5 3) (drill 1.2) (layers *.Cu *.Mask) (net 13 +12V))
  (pad 3 thru_hole oval (at 10 0 270) (size 5 3) (drill 1.2) (layers *.Cu *.Mask) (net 9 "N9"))
  (pad 2 thru_hole oval (at 5 0 270) (size 5 3) (drill 1.2) (layers *.Cu *.Mask) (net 11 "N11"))
  (pad 1 thru_hole oval (at 0 0 270) (size 5 3) (drill 1.2) (layers *.Cu *.Mask) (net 7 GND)))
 (gr_line (start 33.401 58.674) (end 33.401 58.42) (layer B.Cu) (width 0.15))
 (gr_line (start 19.558 75.438) (end 19.558 74.168) (layer Edge.Cuts) (width 0.05))
 (gr_line (start 44.323 75.438) (end 19.558 75.438) (layer Edge.Cuts) (width 0.05))
 (gr_line (start 48.895 19.558) (end 48.895 75.438) (layer Edge.Cuts) (width 0.05))
 (gr_line (start 19.558 19.558) (end 48.895 19.558) (layer Edge.Cuts) (width 0.05))
 (gr_line (start 19.558 74.168) (end 19.558 19.558) (layer Edge.Cuts) (width 0.05))
 (segment (start 31.623 61.148) (end 31.623 62.738) (width 1) (layer B.Cu) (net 9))
 (segment (start 30.513 63.848) (end 30.513 69.088) (width 1) (layer B.Cu) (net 9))
 (segment (start 31.623 62.738) (end 30.513 63.848) (width 1) (layer B.Cu) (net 9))
 (segment (start 25.273 68.848) (end 25.513 69.088) (width 1.2) (layer B.Cu) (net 13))
 (segment (start 25.273 61.468) (end 25.273 68.848) (width 1.2) (layer B.Cu) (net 13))
 (segment (start 25.593 61.148) (end 25.273 61.468) (width 1) (layer B.Cu) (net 13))
 (segment (start 29.083 61.148) (end 25.593 61.148) (width 1) (layer B.Cu) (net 13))
 (segment (start 35.433 61.468) (end 38.923 61.468) (width 1) (layer B.Cu) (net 13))
 (segment (start 35.433 61.468) (end 35.433 62.992) (width 0.8) (layer B.Cu) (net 13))
 (segment (start 35.433 62.992) (end 33.02 65.405) (width 0.8) (layer B.Cu) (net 13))
 (segment (start 33.02 65.405) (end 33.02 71.501) (width 0.8) (layer B.Cu) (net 13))
 (segment (start 33.02 71.501) (end 31.877 72.644) (width 0.8) (layer B.Cu) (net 13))
 (segment (start 29.069 72.644) (end 25.513 69.088) (width 0.8) (layer B.Cu) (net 13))
 (segment (start 31.877 72.644) (end 29.069 72.644) (width 0.8) (layer B.Cu) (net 13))
 (segment (start 40.112 26.323) (end 40.4 26.035) (width 1.2) (layer B.Cu) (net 4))
 (segment (start 40.112 50.162) (end 40.112 26.323) (width 1.2) (layer B.Cu) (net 4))
 (segment (start 35.4 34.674) (end 34.112 35.962) (width 1.2) (layer B.Cu) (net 3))
 (segment (start 35.4 26.035) (end 35.4 34.674) (width 1.2) (layer B.Cu) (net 3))
 (segment (start 30.132 26.303) (end 30.4 26.035) (width 1.2) (layer B.Cu) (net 2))
 (segment (start 30.132 36.754) (end 30.132 26.303) (width 1.2) (layer B.Cu) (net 2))
 (segment (start 25.4 31.316) (end 22.532 34.184) (width 1.2) (layer B.Cu) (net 1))
 (segment (start 25.4 26.035) (end 25.4 31.316) (width 1.2) (layer B.Cu) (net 1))
 (segment (start 43.688 53.594) (end 44.45 53.594) (width 1.2) (layer B.Cu) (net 6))
 (segment (start 46.112 51.932) (end 46.112 48.162) (width 1.2) (layer B.Cu) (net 6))
 (segment (start 44.45 53.594) (end 46.112 51.932) (width 1.2) (layer B.Cu) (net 6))
 (segment (start 40.894 56.388) (end 43.688 53.594) (width 1.2) (layer B.Cu) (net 6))
 (segment (start 35.433 56.388) (end 40.894 56.388) (width 1.2) (layer B.Cu) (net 6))
 (segment (start 25.273 56.388) (end 28.448 56.388) (width 1.2) (layer B.Cu) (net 8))
 (segment (start 30.226 54.61) (end 30.226 53.086) (width 1.2) (layer B.Cu) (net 8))
 (segment (start 28.448 56.388) (end 30.226 54.61) (width 1.2) (layer B.Cu) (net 8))
 (segment (start 30.132 52.992) (end 30.226 53.086) (width 1.2) (layer B.Cu) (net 8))
 (segment (start 30.132 49.424) (end 30.132 52.992) (width 1.2) (layer B.Cu) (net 8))
 (segment (start 35.753 59.248) (end 35.433 58.928) (width 1) (layer B.Cu) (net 12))
 (segment (start 41.402 59.248) (end 38.862 59.248) (width 1) (layer B.Cu) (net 12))
 (segment (start 39.243 59.248) (end 35.753 59.248) (width 1) (layer B.Cu) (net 12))
 (segment (start 25.593 59.248) (end 25.273 58.928) (width 1) (layer B.Cu) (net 10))
 (segment (start 29.083 59.248) (end 25.593 59.248) (width 1) (layer B.Cu) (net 10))
 (segment (start 31.623 59.248) (end 29.083 59.248) (width 1) (layer B.Cu) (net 10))
 (segment (start 35.513 67.738) (end 35.513 69.088) (width 1) (layer B.Cu) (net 11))
 (segment (start 41.021 61.275) (end 41.021 62.611) (width 1) (layer B.Cu) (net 11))
 (segment (start 41.021 62.611) (end 38.481 65.151) (width 1) (layer B.Cu) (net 11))
 (segment (start 38.481 65.151) (end 38.354 65.278) (width 1) (layer B.Cu) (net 11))
 (segment (start 35.513 68.119) (end 35.513 69.088) (width 1) (layer B.Cu) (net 11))
 (segment (start 38.481 65.151) (end 35.513 68.119) (width 1) (layer B.Cu) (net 11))
 (segment (start 46.112 26.747) (end 45.4 26.035) (width 1.2) (layer B.Cu) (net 5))
 (segment (start 46.112 35.962) (end 46.112 26.747) (width 1.2) (layer B.Cu) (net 5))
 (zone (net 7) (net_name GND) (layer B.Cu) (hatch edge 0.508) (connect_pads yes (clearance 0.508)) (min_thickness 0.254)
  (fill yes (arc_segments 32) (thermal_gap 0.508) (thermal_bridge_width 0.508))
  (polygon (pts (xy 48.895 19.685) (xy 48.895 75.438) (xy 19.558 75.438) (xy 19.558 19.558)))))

